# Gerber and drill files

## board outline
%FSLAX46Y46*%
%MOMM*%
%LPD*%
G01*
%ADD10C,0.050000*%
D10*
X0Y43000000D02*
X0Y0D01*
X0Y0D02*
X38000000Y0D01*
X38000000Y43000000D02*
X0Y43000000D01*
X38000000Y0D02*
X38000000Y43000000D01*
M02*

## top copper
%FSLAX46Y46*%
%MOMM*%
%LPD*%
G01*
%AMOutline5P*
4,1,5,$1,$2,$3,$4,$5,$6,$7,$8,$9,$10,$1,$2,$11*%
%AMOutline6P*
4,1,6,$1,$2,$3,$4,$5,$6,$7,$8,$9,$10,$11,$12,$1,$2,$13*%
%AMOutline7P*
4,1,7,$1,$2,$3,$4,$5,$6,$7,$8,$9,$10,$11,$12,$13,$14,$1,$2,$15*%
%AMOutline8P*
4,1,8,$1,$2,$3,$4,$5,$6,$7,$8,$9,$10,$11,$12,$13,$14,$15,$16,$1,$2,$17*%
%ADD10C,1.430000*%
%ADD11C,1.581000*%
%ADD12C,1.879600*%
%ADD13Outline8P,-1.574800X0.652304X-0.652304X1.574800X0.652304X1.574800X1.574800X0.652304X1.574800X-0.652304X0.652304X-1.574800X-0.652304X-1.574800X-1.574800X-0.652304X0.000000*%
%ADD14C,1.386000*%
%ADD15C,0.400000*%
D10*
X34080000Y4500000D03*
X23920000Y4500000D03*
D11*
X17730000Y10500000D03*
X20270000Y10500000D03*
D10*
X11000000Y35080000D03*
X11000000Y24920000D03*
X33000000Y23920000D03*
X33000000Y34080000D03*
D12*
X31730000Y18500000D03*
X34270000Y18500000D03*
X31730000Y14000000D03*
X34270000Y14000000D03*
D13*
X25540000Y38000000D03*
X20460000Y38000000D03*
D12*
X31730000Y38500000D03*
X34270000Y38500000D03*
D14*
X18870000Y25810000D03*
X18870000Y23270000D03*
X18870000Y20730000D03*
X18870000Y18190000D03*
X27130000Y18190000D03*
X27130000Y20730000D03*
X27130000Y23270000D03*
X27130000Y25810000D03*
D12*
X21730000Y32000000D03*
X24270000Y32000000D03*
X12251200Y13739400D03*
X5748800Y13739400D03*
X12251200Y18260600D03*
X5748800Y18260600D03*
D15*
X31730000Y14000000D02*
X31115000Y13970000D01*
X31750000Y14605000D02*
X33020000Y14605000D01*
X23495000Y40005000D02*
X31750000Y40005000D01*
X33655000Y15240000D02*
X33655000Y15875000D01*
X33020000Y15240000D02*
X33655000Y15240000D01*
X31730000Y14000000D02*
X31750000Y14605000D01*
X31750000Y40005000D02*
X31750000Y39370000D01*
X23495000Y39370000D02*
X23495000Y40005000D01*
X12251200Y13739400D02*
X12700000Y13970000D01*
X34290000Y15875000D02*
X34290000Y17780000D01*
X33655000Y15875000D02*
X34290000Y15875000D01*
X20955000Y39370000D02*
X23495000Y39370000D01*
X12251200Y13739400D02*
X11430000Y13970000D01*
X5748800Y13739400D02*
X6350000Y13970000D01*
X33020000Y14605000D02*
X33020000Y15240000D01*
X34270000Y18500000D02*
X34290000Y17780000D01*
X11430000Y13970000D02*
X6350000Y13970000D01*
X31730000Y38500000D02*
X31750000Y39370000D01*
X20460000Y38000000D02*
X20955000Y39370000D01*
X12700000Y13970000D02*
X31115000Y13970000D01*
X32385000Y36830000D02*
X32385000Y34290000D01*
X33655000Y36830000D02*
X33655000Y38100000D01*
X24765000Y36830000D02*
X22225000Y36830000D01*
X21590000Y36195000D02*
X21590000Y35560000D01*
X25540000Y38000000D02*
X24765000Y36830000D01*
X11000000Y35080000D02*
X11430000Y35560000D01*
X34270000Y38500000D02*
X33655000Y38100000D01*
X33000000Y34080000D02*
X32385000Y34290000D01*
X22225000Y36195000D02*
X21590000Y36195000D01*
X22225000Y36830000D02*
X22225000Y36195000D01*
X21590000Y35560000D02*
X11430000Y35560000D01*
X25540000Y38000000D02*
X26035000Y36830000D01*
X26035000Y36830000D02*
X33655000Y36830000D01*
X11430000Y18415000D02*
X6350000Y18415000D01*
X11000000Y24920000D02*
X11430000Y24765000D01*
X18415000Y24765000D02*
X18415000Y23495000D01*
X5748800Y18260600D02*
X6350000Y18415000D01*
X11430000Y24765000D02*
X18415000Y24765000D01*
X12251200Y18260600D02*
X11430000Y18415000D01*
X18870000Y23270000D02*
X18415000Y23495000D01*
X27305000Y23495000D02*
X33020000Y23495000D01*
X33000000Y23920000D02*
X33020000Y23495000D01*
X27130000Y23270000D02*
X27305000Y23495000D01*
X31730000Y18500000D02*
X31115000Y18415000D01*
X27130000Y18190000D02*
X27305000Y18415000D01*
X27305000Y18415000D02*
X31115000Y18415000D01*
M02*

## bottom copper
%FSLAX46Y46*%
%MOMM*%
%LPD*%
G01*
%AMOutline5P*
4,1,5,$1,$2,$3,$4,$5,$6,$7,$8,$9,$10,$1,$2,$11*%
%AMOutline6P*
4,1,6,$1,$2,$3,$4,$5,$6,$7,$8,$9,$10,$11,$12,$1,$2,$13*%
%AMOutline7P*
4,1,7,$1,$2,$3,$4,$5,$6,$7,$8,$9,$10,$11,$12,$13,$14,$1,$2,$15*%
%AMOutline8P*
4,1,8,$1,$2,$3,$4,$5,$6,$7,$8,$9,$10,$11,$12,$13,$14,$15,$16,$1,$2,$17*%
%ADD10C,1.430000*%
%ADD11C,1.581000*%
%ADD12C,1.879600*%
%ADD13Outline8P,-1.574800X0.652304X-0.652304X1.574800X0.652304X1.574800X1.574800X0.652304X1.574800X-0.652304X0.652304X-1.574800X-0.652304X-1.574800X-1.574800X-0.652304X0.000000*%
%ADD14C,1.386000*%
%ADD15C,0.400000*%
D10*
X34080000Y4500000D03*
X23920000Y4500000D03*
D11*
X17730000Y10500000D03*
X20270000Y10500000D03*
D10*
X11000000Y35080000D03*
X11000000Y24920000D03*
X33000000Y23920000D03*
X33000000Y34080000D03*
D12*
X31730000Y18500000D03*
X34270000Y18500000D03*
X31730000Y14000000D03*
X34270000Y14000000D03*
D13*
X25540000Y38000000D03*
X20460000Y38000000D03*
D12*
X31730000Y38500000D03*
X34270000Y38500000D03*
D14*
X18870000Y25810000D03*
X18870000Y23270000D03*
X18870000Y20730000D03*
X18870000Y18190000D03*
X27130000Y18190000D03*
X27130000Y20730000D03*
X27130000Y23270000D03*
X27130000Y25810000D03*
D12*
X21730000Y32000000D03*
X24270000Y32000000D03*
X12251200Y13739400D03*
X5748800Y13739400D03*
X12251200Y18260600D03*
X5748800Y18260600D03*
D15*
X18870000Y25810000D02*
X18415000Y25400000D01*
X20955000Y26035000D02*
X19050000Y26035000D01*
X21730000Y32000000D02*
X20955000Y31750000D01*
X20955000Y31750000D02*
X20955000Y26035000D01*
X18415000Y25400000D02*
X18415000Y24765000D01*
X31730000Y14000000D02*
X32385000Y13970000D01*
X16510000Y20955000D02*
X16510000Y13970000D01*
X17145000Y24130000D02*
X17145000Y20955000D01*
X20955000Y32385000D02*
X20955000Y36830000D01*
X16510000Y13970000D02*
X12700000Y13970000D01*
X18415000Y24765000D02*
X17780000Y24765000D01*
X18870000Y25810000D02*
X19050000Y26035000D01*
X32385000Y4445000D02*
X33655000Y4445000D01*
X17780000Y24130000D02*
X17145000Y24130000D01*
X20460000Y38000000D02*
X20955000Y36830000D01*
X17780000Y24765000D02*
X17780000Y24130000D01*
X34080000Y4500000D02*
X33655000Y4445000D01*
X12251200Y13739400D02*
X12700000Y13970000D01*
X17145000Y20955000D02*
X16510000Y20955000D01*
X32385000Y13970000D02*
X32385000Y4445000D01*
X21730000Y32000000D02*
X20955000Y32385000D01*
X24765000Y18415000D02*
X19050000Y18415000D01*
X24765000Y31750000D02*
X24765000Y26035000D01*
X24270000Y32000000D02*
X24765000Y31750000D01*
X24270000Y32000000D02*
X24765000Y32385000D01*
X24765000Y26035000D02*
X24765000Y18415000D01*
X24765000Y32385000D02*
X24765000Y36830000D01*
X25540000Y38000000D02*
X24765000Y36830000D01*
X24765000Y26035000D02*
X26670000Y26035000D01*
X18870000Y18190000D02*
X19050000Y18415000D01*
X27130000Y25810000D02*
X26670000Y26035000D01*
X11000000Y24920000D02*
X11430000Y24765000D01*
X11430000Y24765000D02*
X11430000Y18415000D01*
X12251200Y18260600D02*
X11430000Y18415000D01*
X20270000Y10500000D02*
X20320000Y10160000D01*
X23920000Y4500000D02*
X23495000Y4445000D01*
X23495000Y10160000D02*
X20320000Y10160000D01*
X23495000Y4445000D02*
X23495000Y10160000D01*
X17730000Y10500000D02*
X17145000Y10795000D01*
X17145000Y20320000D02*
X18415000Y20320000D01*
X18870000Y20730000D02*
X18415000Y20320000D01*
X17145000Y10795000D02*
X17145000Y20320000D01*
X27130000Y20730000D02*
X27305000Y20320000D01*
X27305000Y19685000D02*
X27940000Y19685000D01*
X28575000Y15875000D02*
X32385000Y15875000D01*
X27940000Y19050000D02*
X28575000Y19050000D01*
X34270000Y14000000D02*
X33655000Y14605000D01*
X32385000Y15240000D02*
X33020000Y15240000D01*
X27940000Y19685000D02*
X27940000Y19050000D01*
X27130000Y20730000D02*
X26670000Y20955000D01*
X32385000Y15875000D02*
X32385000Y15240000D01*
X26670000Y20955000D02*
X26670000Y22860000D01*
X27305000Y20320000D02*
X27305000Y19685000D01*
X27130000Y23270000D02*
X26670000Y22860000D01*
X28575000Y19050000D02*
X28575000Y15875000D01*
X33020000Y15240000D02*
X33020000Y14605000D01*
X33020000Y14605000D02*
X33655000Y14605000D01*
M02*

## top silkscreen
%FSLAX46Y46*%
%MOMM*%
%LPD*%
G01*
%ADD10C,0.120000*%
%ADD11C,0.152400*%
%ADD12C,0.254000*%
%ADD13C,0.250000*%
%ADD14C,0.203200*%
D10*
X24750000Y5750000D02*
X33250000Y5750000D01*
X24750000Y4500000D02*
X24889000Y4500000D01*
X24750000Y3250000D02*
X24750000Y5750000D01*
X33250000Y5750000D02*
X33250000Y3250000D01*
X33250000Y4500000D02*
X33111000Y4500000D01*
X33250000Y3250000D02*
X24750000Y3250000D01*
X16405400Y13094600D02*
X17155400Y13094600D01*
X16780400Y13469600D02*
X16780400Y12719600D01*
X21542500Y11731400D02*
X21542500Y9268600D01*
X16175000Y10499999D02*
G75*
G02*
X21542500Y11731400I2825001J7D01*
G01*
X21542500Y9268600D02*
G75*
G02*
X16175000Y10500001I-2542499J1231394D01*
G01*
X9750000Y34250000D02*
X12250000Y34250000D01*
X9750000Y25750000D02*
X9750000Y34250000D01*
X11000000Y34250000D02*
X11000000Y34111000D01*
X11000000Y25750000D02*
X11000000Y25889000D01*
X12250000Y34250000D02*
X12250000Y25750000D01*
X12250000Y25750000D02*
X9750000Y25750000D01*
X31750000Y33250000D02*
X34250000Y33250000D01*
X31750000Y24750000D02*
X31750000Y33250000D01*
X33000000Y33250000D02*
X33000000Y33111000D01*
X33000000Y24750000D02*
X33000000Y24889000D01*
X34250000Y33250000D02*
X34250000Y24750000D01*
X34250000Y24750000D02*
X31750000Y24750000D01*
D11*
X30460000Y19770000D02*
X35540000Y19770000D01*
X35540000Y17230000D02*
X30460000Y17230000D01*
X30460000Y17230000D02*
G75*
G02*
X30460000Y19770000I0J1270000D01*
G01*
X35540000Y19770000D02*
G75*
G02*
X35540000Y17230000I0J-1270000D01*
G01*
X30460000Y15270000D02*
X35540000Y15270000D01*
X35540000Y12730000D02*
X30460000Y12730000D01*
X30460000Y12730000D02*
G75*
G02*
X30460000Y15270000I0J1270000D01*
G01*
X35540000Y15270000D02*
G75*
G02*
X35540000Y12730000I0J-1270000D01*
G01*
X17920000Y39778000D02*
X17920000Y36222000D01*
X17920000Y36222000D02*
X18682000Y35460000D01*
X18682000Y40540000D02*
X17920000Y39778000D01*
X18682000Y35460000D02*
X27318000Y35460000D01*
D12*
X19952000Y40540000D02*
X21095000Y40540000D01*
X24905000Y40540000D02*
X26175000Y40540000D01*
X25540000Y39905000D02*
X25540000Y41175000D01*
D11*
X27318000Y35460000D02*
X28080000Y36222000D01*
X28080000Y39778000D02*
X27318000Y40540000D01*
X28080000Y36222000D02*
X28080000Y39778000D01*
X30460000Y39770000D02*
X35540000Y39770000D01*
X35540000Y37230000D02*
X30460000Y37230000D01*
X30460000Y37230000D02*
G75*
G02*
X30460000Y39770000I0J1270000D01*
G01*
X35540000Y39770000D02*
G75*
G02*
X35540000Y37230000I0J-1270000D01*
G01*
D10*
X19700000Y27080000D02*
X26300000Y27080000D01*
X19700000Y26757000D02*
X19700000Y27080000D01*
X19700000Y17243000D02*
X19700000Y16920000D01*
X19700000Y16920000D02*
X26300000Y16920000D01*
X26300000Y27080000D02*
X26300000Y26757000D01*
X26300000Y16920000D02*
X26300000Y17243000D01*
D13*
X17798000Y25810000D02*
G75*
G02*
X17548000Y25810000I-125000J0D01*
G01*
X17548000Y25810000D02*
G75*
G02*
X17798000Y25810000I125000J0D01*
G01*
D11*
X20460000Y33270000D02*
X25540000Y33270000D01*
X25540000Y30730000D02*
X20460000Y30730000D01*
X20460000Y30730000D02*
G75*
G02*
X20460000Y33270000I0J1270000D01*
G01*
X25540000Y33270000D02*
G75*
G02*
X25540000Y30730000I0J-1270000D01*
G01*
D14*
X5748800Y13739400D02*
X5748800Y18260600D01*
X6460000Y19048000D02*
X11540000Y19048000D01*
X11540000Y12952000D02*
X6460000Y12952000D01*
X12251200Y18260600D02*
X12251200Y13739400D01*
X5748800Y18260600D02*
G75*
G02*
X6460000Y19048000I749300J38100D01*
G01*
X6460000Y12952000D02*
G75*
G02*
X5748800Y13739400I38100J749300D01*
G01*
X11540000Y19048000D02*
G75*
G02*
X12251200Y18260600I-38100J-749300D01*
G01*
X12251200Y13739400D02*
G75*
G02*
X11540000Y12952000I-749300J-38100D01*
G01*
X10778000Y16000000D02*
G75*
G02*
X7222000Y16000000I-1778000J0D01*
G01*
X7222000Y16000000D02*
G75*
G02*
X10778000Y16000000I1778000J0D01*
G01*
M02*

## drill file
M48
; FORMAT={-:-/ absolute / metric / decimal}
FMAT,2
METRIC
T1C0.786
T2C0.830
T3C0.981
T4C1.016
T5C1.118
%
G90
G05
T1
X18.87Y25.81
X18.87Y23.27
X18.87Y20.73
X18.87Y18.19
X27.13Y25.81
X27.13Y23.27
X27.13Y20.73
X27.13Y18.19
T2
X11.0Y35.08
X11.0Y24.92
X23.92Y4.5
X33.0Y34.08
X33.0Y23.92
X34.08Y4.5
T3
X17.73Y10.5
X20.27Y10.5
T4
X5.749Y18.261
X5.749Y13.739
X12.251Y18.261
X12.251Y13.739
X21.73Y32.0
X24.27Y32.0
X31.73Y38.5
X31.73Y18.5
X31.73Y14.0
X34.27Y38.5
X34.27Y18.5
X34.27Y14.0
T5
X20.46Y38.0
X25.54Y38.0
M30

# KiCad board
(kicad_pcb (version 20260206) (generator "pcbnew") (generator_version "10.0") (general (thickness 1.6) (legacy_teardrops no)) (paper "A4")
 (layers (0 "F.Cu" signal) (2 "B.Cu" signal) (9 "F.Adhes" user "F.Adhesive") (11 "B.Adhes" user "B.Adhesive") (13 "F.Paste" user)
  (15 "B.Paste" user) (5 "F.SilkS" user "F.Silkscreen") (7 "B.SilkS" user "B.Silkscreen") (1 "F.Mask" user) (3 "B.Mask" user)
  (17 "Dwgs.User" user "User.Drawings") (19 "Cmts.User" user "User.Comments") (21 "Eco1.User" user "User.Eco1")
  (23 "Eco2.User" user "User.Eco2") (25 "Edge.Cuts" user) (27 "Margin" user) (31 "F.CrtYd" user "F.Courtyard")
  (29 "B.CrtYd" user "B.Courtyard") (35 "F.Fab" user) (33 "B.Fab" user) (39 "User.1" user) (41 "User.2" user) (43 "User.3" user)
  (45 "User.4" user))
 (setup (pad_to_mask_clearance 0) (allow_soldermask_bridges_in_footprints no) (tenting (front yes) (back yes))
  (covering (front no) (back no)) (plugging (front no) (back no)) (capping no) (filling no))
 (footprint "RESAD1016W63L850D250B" (layer "F.Cu") (at 29 -4.5 180)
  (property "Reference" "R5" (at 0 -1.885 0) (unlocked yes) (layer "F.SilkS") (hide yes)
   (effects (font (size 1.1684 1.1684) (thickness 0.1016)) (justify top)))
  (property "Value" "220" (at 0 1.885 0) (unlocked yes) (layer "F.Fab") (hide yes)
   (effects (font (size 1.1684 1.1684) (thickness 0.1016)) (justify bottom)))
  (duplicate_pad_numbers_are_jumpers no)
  (fp_line (start 4.25 1.25) (end -4.25 1.25) (stroke (width 0.12) (type solid)) (layer "F.SilkS"))
  (fp_line (start 4.25 0) (end 4.111 0) (stroke (width 0.12) (type solid)) (layer "F.SilkS"))
  (fp_line (start 4.25 -1.25) (end 4.25 1.25) (stroke (width 0.12) (type solid)) (layer "F.SilkS"))
  (fp_line (start -4.25 1.25) (end -4.25 -1.25) (stroke (width 0.12) (type solid)) (layer "F.SilkS"))
  (fp_line (start -4.25 0) (end -4.111 0) (stroke (width 0.12) (type solid)) (layer "F.SilkS"))
  (fp_line (start -4.25 -1.25) (end 4.25 -1.25) (stroke (width 0.12) (type solid)) (layer "F.SilkS"))
  (pad "1" thru_hole circle (at -5.08 0 180) (size 1.43 1.43) (drill 0.83) (layers "*.Cu" "*.Mask") (remove_unused_layers no) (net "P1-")
   (solder_mask_margin 0.1016) (thermal_bridge_angle 0))
  (pad "2" thru_hole circle (at 5.08 0 180) (size 1.43 1.43) (drill 0.83) (layers "*.Cu" "*.Mask") (remove_unused_layers no) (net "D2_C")
   (solder_mask_margin 0.1016) (thermal_bridge_angle 0)))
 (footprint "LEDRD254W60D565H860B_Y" (layer "F.Cu") (at 19 -10.5)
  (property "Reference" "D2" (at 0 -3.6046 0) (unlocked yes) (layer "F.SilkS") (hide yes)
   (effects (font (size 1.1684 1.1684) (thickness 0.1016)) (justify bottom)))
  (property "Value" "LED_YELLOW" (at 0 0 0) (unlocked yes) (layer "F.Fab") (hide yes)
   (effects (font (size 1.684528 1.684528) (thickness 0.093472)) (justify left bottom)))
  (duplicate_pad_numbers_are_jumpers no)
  (fp_line (start -2.5946 -2.5946) (end -1.8446 -2.5946) (stroke (width 0.12) (type solid)) (layer "F.SilkS"))
  (fp_line (start -2.2196 -2.9696) (end -2.2196 -2.2196) (stroke (width 0.12) (type solid)) (layer "F.SilkS"))
  (fp_line (start 2.5425 -1.2314) (end 2.5425 1.2314) (stroke (width 0.12) (type solid)) (layer "F.SilkS"))
  (fp_arc (start -2.825 0.000001) (mid -0.631694 -2.753475) (end 2.5425 -1.2314) (stroke (width 0.12) (type solid)) (layer "F.SilkS"))
  (fp_arc (start 2.5425 1.2314) (mid -0.631694 2.753475) (end -2.825 -0.000001) (stroke (width 0.12) (type solid)) (layer "F.SilkS"))
  (pad "1" thru_hole circle (at -1.27 0) (size 1.581 1.581) (drill 0.981) (layers "*.Cu" "*.Mask") (remove_unused_layers no) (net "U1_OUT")
   (solder_mask_margin 0.1016) (thermal_bridge_angle 0))
  (pad "2" thru_hole circle (at 1.27 0) (size 1.581 1.581) (drill 0.981) (layers "*.Cu" "*.Mask") (remove_unused_layers no) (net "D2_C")
   (solder_mask_margin 0.1016) (thermal_bridge_angle 0)))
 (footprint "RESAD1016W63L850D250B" (layer "F.Cu") (at 11 -30 -90)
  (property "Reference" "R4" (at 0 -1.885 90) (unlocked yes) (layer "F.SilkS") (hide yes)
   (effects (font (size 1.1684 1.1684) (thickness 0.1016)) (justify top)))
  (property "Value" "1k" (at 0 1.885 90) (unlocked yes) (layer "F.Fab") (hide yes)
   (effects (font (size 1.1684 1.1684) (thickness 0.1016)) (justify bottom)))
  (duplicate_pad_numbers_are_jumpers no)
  (fp_line (start -4.25 1.25) (end -4.25 -1.25) (stroke (width 0.12) (type solid)) (layer "F.SilkS"))
  (fp_line (start 4.25 1.25) (end -4.25 1.25) (stroke (width 0.12) (type solid)) (layer "F.SilkS"))
  (fp_line (start -4.25 0) (end -4.111 0) (stroke (width 0.12) (type solid)) (layer "F.SilkS"))
  (fp_line (start 4.25 0) (end 4.111 0) (stroke (width 0.12) (type solid)) (layer "F.SilkS"))
  (fp_line (start -4.25 -1.25) (end 4.25 -1.25) (stroke (width 0.12) (type solid)) (layer "F.SilkS"))
  (fp_line (start 4.25 -1.25) (end 4.25 1.25) (stroke (width 0.12) (type solid)) (layer "F.SilkS"))
  (pad "1" thru_hole circle (at -5.08 0 270) (size 1.43 1.43) (drill 0.83) (layers "*.Cu" "*.Mask") (remove_unused_layers no) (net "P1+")
   (solder_mask_margin 0.1016) (thermal_bridge_angle 0))
  (pad "2" thru_hole circle (at 5.08 0 270) (size 1.43 1.43) (drill 0.83) (layers "*.Cu" "*.Mask") (remove_unused_layers no) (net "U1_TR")
   (solder_mask_margin 0.1016) (thermal_bridge_angle 0)))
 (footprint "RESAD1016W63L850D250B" (layer "F.Cu") (at 33 -29 90)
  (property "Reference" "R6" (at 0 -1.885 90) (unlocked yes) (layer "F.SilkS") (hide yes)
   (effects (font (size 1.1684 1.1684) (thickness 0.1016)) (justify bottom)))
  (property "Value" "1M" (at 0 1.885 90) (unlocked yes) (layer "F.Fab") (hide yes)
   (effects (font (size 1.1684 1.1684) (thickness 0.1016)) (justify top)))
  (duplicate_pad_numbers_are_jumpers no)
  (fp_line (start 4.25 -1.25) (end 4.25 1.25) (stroke (width 0.12) (type solid)) (layer "F.SilkS"))
  (fp_line (start -4.25 -1.25) (end 4.25 -1.25) (stroke (width 0.12) (type solid)) (layer "F.SilkS"))
  (fp_line (start 4.25 0) (end 4.111 0) (stroke (width 0.12) (type solid)) (layer "F.SilkS"))
  (fp_line (start -4.25 0) (end -4.111 0) (stroke (width 0.12) (type solid)) (layer "F.SilkS"))
  (fp_line (start 4.25 1.25) (end -4.25 1.25) (stroke (width 0.12) (type solid)) (layer "F.SilkS"))
  (fp_line (start -4.25 1.25) (end -4.25 -1.25) (stroke (width 0.12) (type solid)) (layer "F.SilkS"))
  (pad "1" thru_hole circle (at -5.08 0 90) (size 1.43 1.43) (drill 0.83) (layers "*.Cu" "*.Mask") (remove_unused_layers no) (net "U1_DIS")
   (solder_mask_margin 0.1016) (thermal_bridge_angle 0))
  (pad "2" thru_hole circle (at 5.08 0 90) (size 1.43 1.43) (drill 0.83) (layers "*.Cu" "*.Mask") (remove_unused_layers no) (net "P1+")
   (solder_mask_margin 0.1016) (thermal_bridge_angle 0)))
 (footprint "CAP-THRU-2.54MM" (layer "F.Cu") (at 33 -18.5)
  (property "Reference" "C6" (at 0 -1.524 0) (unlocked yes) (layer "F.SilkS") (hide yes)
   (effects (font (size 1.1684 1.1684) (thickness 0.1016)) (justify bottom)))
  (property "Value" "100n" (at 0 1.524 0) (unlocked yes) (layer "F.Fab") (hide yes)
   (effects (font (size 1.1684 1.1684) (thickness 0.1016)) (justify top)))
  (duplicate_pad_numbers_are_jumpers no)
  (fp_line (start -2.54 -1.27) (end 2.54 -1.27) (stroke (width 0.1524) (type solid)) (layer "F.SilkS"))
  (fp_line (start 2.54 1.27) (end -2.54 1.27) (stroke (width 0.1524) (type solid)) (layer "F.SilkS"))
  (fp_arc (start -2.54 1.27) (mid -3.81 0) (end -2.54 -1.27) (stroke (width 0.1524) (type solid)) (layer "F.SilkS"))
  (fp_arc (start 2.54 -1.27) (mid 3.81 0) (end 2.54 1.27) (stroke (width 0.1524) (type solid)) (layer "F.SilkS"))
  (pad "1" thru_hole circle (at -1.27 0) (size 1.8796 1.8796) (drill 1.016) (layers "*.Cu" "*.Mask") (remove_unused_layers no) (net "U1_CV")
   (solder_mask_margin 0.1016) (thermal_bridge_angle 0))
  (pad "2" thru_hole circle (at 1.27 0) (size 1.8796 1.8796) (drill 1.016) (layers "*.Cu" "*.Mask") (remove_unused_layers no) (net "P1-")
   (solder_mask_margin 0.1016) (thermal_bridge_angle 0)))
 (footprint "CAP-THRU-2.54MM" (layer "F.Cu") (at 33 -14)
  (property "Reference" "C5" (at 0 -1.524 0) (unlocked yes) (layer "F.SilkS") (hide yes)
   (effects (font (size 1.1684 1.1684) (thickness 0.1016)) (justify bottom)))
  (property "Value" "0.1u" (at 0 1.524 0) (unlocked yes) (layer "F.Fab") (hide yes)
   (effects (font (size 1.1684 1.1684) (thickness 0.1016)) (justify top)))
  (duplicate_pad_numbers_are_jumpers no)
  (fp_line (start -2.54 -1.27) (end 2.54 -1.27) (stroke (width 0.1524) (type solid)) (layer "F.SilkS"))
  (fp_line (start 2.54 1.27) (end -2.54 1.27) (stroke (width 0.1524) (type solid)) (layer "F.SilkS"))
  (fp_arc (start -2.54 1.27) (mid -3.81 0) (end -2.54 -1.27) (stroke (width 0.1524) (type solid)) (layer "F.SilkS"))
  (fp_arc (start 2.54 -1.27) (mid 3.81 0) (end 2.54 1.27) (stroke (width 0.1524) (type solid)) (layer "F.SilkS"))
  (pad "1" thru_hole circle (at -1.27 0) (size 1.8796 1.8796) (drill 1.016) (layers "*.Cu" "*.Mask") (remove_unused_layers no) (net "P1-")
   (solder_mask_margin 0.1016) (thermal_bridge_angle 0))
  (pad "2" thru_hole circle (at 1.27 0) (size 1.8796 1.8796) (drill 1.016) (layers "*.Cu" "*.Mask") (remove_unused_layers no) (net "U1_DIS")
   (solder_mask_margin 0.1016) (thermal_bridge_angle 0)))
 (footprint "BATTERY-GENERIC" (layer "F.Cu") (at 23 -38)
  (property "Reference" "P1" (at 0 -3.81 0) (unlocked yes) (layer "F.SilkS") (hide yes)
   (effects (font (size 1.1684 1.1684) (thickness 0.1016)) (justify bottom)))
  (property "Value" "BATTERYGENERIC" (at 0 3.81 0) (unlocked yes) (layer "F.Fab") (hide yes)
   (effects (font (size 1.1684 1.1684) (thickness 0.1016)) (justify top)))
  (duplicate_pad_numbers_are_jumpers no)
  (fp_line (start -5.08 -1.778) (end -5.08 1.778) (stroke (width 0.1524) (type solid)) (layer "F.SilkS"))
  (fp_line (start -5.08 1.778) (end -4.318 2.54) (stroke (width 0.1524) (type solid)) (layer "F.SilkS"))
  (fp_line (start -4.318 -2.54) (end -5.08 -1.778) (stroke (width 0.1524) (type solid)) (layer "F.SilkS"))
  (fp_line (start -4.318 2.54) (end 4.318 2.54) (stroke (width 0.1524) (type solid)) (layer "F.SilkS"))
  (fp_line (start -3.048 -2.54) (end -1.905 -2.54) (stroke (width 0.254) (type solid)) (layer "F.SilkS"))
  (fp_line (start 1.905 -2.54) (end 3.175 -2.54) (stroke (width 0.254) (type solid)) (layer "F.SilkS"))
  (fp_line (start 2.54 -1.905) (end 2.54 -3.175) (stroke (width 0.254) (type solid)) (layer "F.SilkS"))
  (fp_line (start 4.318 2.54) (end 5.08 1.778) (stroke (width 0.1524) (type solid)) (layer "F.SilkS"))
  (fp_line (start 5.08 -1.778) (end 4.318 -2.54) (stroke (width 0.1524) (type solid)) (layer "F.SilkS"))
  (fp_line (start 5.08 1.778) (end 5.08 -1.778) (stroke (width 0.1524) (type solid)) (layer "F.SilkS"))
  (pad "+" thru_hole roundrect (at 2.54 0) (size 3.1496 3.1496) (drill 1.1176) (layers "*.Cu" "*.Mask") (remove_unused_layers no)
   (roundrect_rratio 0.25) (chamfer_ratio 0.2928932188) (chamfer top_left top_right bottom_left bottom_right) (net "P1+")
   (solder_mask_margin 0.1016) (thermal_bridge_angle 0))
  (pad "-" thru_hole roundrect (at -2.54 0) (size 3.1496 3.1496) (drill 1.1176) (layers "*.Cu" "*.Mask") (remove_unused_layers no)
   (roundrect_rratio 0.25) (chamfer_ratio 0.2928932188) (chamfer top_left top_right bottom_left bottom_right) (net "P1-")
   (solder_mask_margin 0.1016) (thermal_bridge_angle 0)))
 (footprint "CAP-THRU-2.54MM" (layer "F.Cu") (at 33 -38.5)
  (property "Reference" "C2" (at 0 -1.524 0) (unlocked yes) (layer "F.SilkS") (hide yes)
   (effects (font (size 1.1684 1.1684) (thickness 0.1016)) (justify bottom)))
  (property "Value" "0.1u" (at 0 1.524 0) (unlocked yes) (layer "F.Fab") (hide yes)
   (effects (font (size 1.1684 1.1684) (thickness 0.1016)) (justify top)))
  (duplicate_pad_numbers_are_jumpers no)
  (fp_line (start -2.54 -1.27) (end 2.54 -1.27) (stroke (width 0.1524) (type solid)) (layer "F.SilkS"))
  (fp_line (start 2.54 1.27) (end -2.54 1.27) (stroke (width 0.1524) (type solid)) (layer "F.SilkS"))
  (fp_arc (start -2.54 1.27) (mid -3.81 0) (end -2.54 -1.27) (stroke (width 0.1524) (type solid)) (layer "F.SilkS"))
  (fp_arc (start 2.54 -1.27) (mid 3.81 0) (end 2.54 1.27) (stroke (width 0.1524) (type solid)) (layer "F.SilkS"))
  (pad "1" thru_hole circle (at -1.27 0) (size 1.8796 1.8796) (drill 1.016) (layers "*.Cu" "*.Mask") (remove_unused_layers no) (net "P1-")
   (solder_mask_margin 0.1016) (thermal_bridge_angle 0))
  (pad "2" thru_hole circle (at 1.27 0) (size 1.8796 1.8796) (drill 1.016) (layers "*.Cu" "*.Mask") (remove_unused_layers no) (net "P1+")
   (solder_mask_margin 0.1016) (thermal_bridge_angle 0)))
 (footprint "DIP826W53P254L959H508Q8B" (layer "F.Cu") (at 23 -22)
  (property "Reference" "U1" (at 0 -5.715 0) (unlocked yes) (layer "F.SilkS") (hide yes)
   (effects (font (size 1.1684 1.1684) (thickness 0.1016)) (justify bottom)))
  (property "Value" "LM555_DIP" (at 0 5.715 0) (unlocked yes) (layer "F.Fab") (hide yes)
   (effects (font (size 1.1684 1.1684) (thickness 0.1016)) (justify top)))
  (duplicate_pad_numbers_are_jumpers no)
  (fp_line (start -3.3 -5.08) (end 3.3 -5.08) (stroke (width 0.12) (type solid)) (layer "F.SilkS"))
  (fp_line (start -3.3 -4.757) (end -3.3 -5.08) (stroke (width 0.12) (type solid)) (layer "F.SilkS"))
  (fp_line (start -3.3 4.757) (end -3.3 5.08) (stroke (width 0.12) (type solid)) (layer "F.SilkS"))
  (fp_line (start -3.3 5.08) (end 3.3 5.08) (stroke (width 0.12) (type solid)) (layer "F.SilkS"))
  (fp_line (start 3.3 -5.08) (end 3.3 -4.757) (stroke (width 0.12) (type solid)) (layer "F.SilkS"))
  (fp_line (start 3.3 5.08) (end 3.3 4.757) (stroke (width 0.12) (type solid)) (layer "F.SilkS"))
  (fp_circle (center -5.327 -3.81) (end -5.202 -3.81) (stroke (width 0.25) (type solid)) (fill yes) (layer "F.SilkS"))
  (pad "1" thru_hole circle (at -4.13 -3.81) (size 1.386 1.386) (drill 0.786) (layers "*.Cu" "*.Mask") (remove_unused_layers no) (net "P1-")
   (solder_mask_margin 0.1016) (thermal_bridge_angle 0))
  (pad "2" thru_hole circle (at -4.13 -1.27) (size 1.386 1.386) (drill 0.786) (layers "*.Cu" "*.Mask") (remove_unused_layers no)
   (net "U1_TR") (solder_mask_margin 0.1016) (thermal_bridge_angle 0))
  (pad "3" thru_hole circle (at -4.13 1.27) (size 1.386 1.386) (drill 0.786) (layers "*.Cu" "*.Mask") (remove_unused_layers no)
   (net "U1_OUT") (solder_mask_margin 0.1016) (thermal_bridge_angle 0))
  (pad "4" thru_hole circle (at -4.13 3.81) (size 1.386 1.386) (drill 0.786) (layers "*.Cu" "*.Mask") (remove_unused_layers no) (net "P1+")
   (solder_mask_margin 0.1016) (thermal_bridge_angle 0))
  (pad "5" thru_hole circle (at 4.13 3.81) (size 1.386 1.386) (drill 0.786) (layers "*.Cu" "*.Mask") (remove_unused_layers no) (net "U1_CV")
   (solder_mask_margin 0.1016) (thermal_bridge_angle 0))
  (pad "6" thru_hole circle (at 4.13 1.27) (size 1.386 1.386) (drill 0.786) (layers "*.Cu" "*.Mask") (remove_unused_layers no)
   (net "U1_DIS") (solder_mask_margin 0.1016) (thermal_bridge_angle 0))
  (pad "7" thru_hole circle (at 4.13 -1.27) (size 1.386 1.386) (drill 0.786) (layers "*.Cu" "*.Mask") (remove_unused_layers no)
   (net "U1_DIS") (solder_mask_margin 0.1016) (thermal_bridge_angle 0))
  (pad "8" thru_hole circle (at 4.13 -3.81) (size 1.386 1.386) (drill 0.786) (layers "*.Cu" "*.Mask") (remove_unused_layers no) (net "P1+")
   (solder_mask_margin 0.1016) (thermal_bridge_angle 0)))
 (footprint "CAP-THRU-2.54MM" (layer "F.Cu") (at 23 -32)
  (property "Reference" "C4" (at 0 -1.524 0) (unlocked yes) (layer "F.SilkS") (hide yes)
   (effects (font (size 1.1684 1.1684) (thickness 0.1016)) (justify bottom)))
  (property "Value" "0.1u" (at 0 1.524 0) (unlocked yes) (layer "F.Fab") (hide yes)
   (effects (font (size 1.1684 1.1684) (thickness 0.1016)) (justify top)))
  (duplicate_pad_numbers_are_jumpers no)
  (fp_line (start -2.54 -1.27) (end 2.54 -1.27) (stroke (width 0.1524) (type solid)) (layer "F.SilkS"))
  (fp_line (start 2.54 1.27) (end -2.54 1.27) (stroke (width 0.1524) (type solid)) (layer "F.SilkS"))
  (fp_arc (start -2.54 1.27) (mid -3.81 0) (end -2.54 -1.27) (stroke (width 0.1524) (type solid)) (layer "F.SilkS"))
  (fp_arc (start 2.54 -1.27) (mid 3.81 0) (end 2.54 1.27) (stroke (width 0.1524) (type solid)) (layer "F.SilkS"))
  (pad "1" thru_hole circle (at -1.27 0) (size 1.8796 1.8796) (drill 1.016) (layers "*.Cu" "*.Mask") (remove_unused_layers no) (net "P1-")
   (solder_mask_margin 0.1016) (thermal_bridge_angle 0))
  (pad "2" thru_hole circle (at 1.27 0) (size 1.8796 1.8796) (drill 1.016) (layers "*.Cu" "*.Mask") (remove_unused_layers no) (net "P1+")
   (solder_mask_margin 0.1016) (thermal_bridge_angle 0)))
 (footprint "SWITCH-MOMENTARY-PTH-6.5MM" (layer "F.Cu") (at 9 -16 180)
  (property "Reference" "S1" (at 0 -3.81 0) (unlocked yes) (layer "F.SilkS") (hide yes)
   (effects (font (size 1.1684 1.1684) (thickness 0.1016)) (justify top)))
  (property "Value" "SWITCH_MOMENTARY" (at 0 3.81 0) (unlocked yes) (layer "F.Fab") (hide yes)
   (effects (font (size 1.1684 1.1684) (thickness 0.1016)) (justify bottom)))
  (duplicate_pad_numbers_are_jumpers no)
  (fp_line (start 3.2512 -2.2606) (end 3.2512 2.2606) (stroke (width 0.2032) (type solid)) (layer "F.SilkS"))
  (fp_line (start 2.54 3.048) (end -2.54 3.048) (stroke (width 0.2032) (type solid)) (layer "F.SilkS"))
  (fp_line (start -2.54 -3.048) (end 2.54 -3.048) (stroke (width 0.2032) (type solid)) (layer "F.SilkS"))
  (fp_line (start -3.2512 2.2606) (end -3.2512 -2.2606) (stroke (width 0.2032) (type solid)) (layer "F.SilkS"))
  (fp_arc (start 3.2512 2.2606) (mid 3.058676 2.801594) (end 2.54 3.048) (stroke (width 0.2032) (type solid)) (layer "F.SilkS"))
  (fp_arc (start 2.54 -3.048) (mid 3.058676 -2.801594) (end 3.2512 -2.2606) (stroke (width 0.2032) (type solid)) (layer "F.SilkS"))
  (fp_arc (start -2.54 3.048) (mid -3.058676 2.801594) (end -3.2512 2.2606) (stroke (width 0.2032) (type solid)) (layer "F.SilkS"))
  (fp_arc (start -3.2512 -2.2606) (mid -3.058676 -2.801594) (end -2.54 -3.048) (stroke (width 0.2032) (type solid)) (layer "F.SilkS"))
  (fp_circle (center 0 0) (end 1.778 0) (stroke (width 0.2032) (type solid)) (fill no) (layer "F.SilkS"))
  (pad "1" thru_hole circle (at -3.2512 -2.2606 180) (size 1.8796 1.8796) (drill 1.016) (layers "*.Cu" "*.Mask") (remove_unused_layers no)
   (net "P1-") (solder_mask_margin 0.1016) (thermal_bridge_angle 0))
  (pad "2" thru_hole circle (at 3.2512 -2.2606 180) (size 1.8796 1.8796) (drill 1.016) (layers "*.Cu" "*.Mask") (remove_unused_layers no)
   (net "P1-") (solder_mask_margin 0.1016) (thermal_bridge_angle 0))
  (pad "3" thru_hole circle (at -3.2512 2.2606 180) (size 1.8796 1.8796) (drill 1.016) (layers "*.Cu" "*.Mask") (remove_unused_layers no)
   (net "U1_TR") (solder_mask_margin 0.1016) (thermal_bridge_angle 0))
  (pad "4" thru_hole circle (at 3.2512 2.2606 180) (size 1.8796 1.8796) (drill 1.016) (layers "*.Cu" "*.Mask") (remove_unused_layers no)
   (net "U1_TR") (solder_mask_margin 0.1016) (thermal_bridge_angle 0)))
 (gr_line (start 0 -43) (end 0 0) (stroke (width 0.05) (type solid)) (layer "Edge.Cuts"))
 (gr_line (start 0 0) (end 38 0) (stroke (width 0.05) (type solid)) (layer "Edge.Cuts"))
 (gr_line (start 38 -43) (end 0 -43) (stroke (width 0.05) (type solid)) (layer "Edge.Cuts"))
 (gr_line (start 38 0) (end 38 -43) (stroke (width 0.05) (type solid)) (layer "Edge.Cuts"))
 (segment (start 31.73 -14) (end 31.115 -13.97) (width 0.4) (layer "F.Cu") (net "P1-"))
 (segment (start 31.75 -14.605) (end 33.02 -14.605) (width 0.4) (layer "F.Cu") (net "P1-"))
 (segment (start 23.495 -40.005) (end 31.75 -40.005) (width 0.4) (layer "F.Cu") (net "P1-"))
 (segment (start 33.655 -15.24) (end 33.655 -15.875) (width 0.4) (layer "F.Cu") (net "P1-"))
 (segment (start 33.02 -15.24) (end 33.655 -15.24) (width 0.4) (layer "F.Cu") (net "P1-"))
 (segment (start 31.73 -14) (end 31.75 -14.605) (width 0.4) (layer "F.Cu") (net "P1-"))
 (segment (start 31.75 -40.005) (end 31.75 -39.37) (width 0.4) (layer "F.Cu") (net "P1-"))
 (segment (start 23.495 -39.37) (end 23.495 -40.005) (width 0.4) (layer "F.Cu") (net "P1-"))
 (segment (start 12.2512 -13.7394) (end 12.7 -13.97) (width 0.4) (layer "F.Cu") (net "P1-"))
 (segment (start 34.29 -15.875) (end 34.29 -17.78) (width 0.4) (layer "F.Cu") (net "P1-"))
 (segment (start 33.655 -15.875) (end 34.29 -15.875) (width 0.4) (layer "F.Cu") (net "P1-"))
 (segment (start 20.955 -39.37) (end 23.495 -39.37) (width 0.4) (layer "F.Cu") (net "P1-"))
 (segment (start 12.2512 -13.7394) (end 11.43 -13.97) (width 0.4) (layer "F.Cu") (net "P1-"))
 (segment (start 5.7488 -13.7394) (end 6.35 -13.97) (width 0.4) (layer "F.Cu") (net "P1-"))
 (segment (start 33.02 -14.605) (end 33.02 -15.24) (width 0.4) (layer "F.Cu") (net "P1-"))
 (segment (start 34.27 -18.5) (end 34.29 -17.78) (width 0.4) (layer "F.Cu") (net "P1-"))
 (segment (start 11.43 -13.97) (end 6.35 -13.97) (width 0.4) (layer "F.Cu") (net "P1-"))
 (segment (start 31.73 -38.5) (end 31.75 -39.37) (width 0.4) (layer "F.Cu") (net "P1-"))
 (segment (start 20.46 -38) (end 20.955 -39.37) (width 0.4) (layer "F.Cu") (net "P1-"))
 (segment (start 12.7 -13.97) (end 31.115 -13.97) (width 0.4) (layer "F.Cu") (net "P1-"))
 (segment (start 18.87 -25.81) (end 18.415 -25.4) (width 0.4) (layer "B.Cu") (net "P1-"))
 (segment (start 20.955 -26.035) (end 19.05 -26.035) (width 0.4) (layer "B.Cu") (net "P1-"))
 (segment (start 21.73 -32) (end 20.955 -31.75) (width 0.4) (layer "B.Cu") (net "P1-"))
 (segment (start 20.955 -31.75) (end 20.955 -26.035) (width 0.4) (layer "B.Cu") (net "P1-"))
 (segment (start 18.415 -25.4) (end 18.415 -24.765) (width 0.4) (layer "B.Cu") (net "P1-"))
 (segment (start 31.73 -14) (end 32.385 -13.97) (width 0.4) (layer "B.Cu") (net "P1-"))
 (segment (start 16.51 -20.955) (end 16.51 -13.97) (width 0.4) (layer "B.Cu") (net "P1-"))
 (segment (start 17.145 -24.13) (end 17.145 -20.955) (width 0.4) (layer "B.Cu") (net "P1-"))
 (segment (start 20.955 -32.385) (end 20.955 -36.83) (width 0.4) (layer "B.Cu") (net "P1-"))
 (segment (start 16.51 -13.97) (end 12.7 -13.97) (width 0.4) (layer "B.Cu") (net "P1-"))
 (segment (start 18.415 -24.765) (end 17.78 -24.765) (width 0.4) (layer "B.Cu") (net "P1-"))
 (segment (start 18.87 -25.81) (end 19.05 -26.035) (width 0.4) (layer "B.Cu") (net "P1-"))
 (segment (start 32.385 -4.445) (end 33.655 -4.445) (width 0.4) (layer "B.Cu") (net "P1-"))
 (segment (start 17.78 -24.13) (end 17.145 -24.13) (width 0.4) (layer "B.Cu") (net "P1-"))
 (segment (start 20.46 -38) (end 20.955 -36.83) (width 0.4) (layer "B.Cu") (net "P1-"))
 (segment (start 17.78 -24.765) (end 17.78 -24.13) (width 0.4) (layer "B.Cu") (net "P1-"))
 (segment (start 34.08 -4.5) (end 33.655 -4.445) (width 0.4) (layer "B.Cu") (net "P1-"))
 (segment (start 12.2512 -13.7394) (end 12.7 -13.97) (width 0.4) (layer "B.Cu") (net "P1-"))
 (segment (start 17.145 -20.955) (end 16.51 -20.955) (width 0.4) (layer "B.Cu") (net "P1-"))
 (segment (start 32.385 -13.97) (end 32.385 -4.445) (width 0.4) (layer "B.Cu") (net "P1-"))
 (segment (start 21.73 -32) (end 20.955 -32.385) (width 0.4) (layer "B.Cu") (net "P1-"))
 (segment (start 32.385 -36.83) (end 32.385 -34.29) (width 0.4) (layer "F.Cu") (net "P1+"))
 (segment (start 33.655 -36.83) (end 33.655 -38.1) (width 0.4) (layer "F.Cu") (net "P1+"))
 (segment (start 24.765 -36.83) (end 22.225 -36.83) (width 0.4) (layer "F.Cu") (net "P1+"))
 (segment (start 21.59 -36.195) (end 21.59 -35.56) (width 0.4) (layer "F.Cu") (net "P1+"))
 (segment (start 25.54 -38) (end 24.765 -36.83) (width 0.4) (layer "F.Cu") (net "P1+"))
 (segment (start 11 -35.08) (end 11.43 -35.56) (width 0.4) (layer "F.Cu") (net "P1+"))
 (segment (start 34.27 -38.5) (end 33.655 -38.1) (width 0.4) (layer "F.Cu") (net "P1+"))
 (segment (start 33 -34.08) (end 32.385 -34.29) (width 0.4) (layer "F.Cu") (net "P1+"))
 (segment (start 22.225 -36.195) (end 21.59 -36.195) (width 0.4) (layer "F.Cu") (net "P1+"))
 (segment (start 22.225 -36.83) (end 22.225 -36.195) (width 0.4) (layer "F.Cu") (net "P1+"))
 (segment (start 21.59 -35.56) (end 11.43 -35.56) (width 0.4) (layer "F.Cu") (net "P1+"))
 (segment (start 25.54 -38) (end 26.035 -36.83) (width 0.4) (layer "F.Cu") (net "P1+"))
 (segment (start 26.035 -36.83) (end 33.655 -36.83) (width 0.4) (layer "F.Cu") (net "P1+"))
 (segment (start 24.765 -18.415) (end 19.05 -18.415) (width 0.4) (layer "B.Cu") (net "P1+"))
 (segment (start 24.765 -31.75) (end 24.765 -26.035) (width 0.4) (layer "B.Cu") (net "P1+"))
 (segment (start 24.27 -32) (end 24.765 -31.75) (width 0.4) (layer "B.Cu") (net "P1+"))
 (segment (start 24.27 -32) (end 24.765 -32.385) (width 0.4) (layer "B.Cu") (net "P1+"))
 (segment (start 24.765 -26.035) (end 24.765 -18.415) (width 0.4) (layer "B.Cu") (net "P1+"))
 (segment (start 24.765 -32.385) (end 24.765 -36.83) (width 0.4) (layer "B.Cu") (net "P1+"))
 (segment (start 25.54 -38) (end 24.765 -36.83) (width 0.4) (layer "B.Cu") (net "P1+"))
 (segment (start 24.765 -26.035) (end 26.67 -26.035) (width 0.4) (layer "B.Cu") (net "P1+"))
 (segment (start 18.87 -18.19) (end 19.05 -18.415) (width 0.4) (layer "B.Cu") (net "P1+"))
 (segment (start 27.13 -25.81) (end 26.67 -26.035) (width 0.4) (layer "B.Cu") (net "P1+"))
 (segment (start 11.43 -18.415) (end 6.35 -18.415) (width 0.4) (layer "F.Cu") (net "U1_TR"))
 (segment (start 11 -24.92) (end 11.43 -24.765) (width 0.4) (layer "F.Cu") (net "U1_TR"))
 (segment (start 18.415 -24.765) (end 18.415 -23.495) (width 0.4) (layer "F.Cu") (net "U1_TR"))
 (segment (start 5.7488 -18.2606) (end 6.35 -18.415) (width 0.4) (layer "F.Cu") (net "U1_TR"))
 (segment (start 11.43 -24.765) (end 18.415 -24.765) (width 0.4) (layer "F.Cu") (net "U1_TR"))
 (segment (start 12.2512 -18.2606) (end 11.43 -18.415) (width 0.4) (layer "F.Cu") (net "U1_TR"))
 (segment (start 18.87 -23.27) (end 18.415 -23.495) (width 0.4) (layer "F.Cu") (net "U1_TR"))
 (segment (start 11 -24.92) (end 11.43 -24.765) (width 0.4) (layer "B.Cu") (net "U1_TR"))
 (segment (start 11.43 -24.765) (end 11.43 -18.415) (width 0.4) (layer "B.Cu") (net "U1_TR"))
 (segment (start 12.2512 -18.2606) (end 11.43 -18.415) (width 0.4) (layer "B.Cu") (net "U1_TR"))
 (segment (start 20.27 -10.5) (end 20.32 -10.16) (width 0.4) (layer "B.Cu") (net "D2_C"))
 (segment (start 23.92 -4.5) (end 23.495 -4.445) (width 0.4) (layer "B.Cu") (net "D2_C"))
 (segment (start 23.495 -10.16) (end 20.32 -10.16) (width 0.4) (layer "B.Cu") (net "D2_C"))
 (segment (start 23.495 -4.445) (end 23.495 -10.16) (width 0.4) (layer "B.Cu") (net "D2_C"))
 (segment (start 17.73 -10.5) (end 17.145 -10.795) (width 0.4) (layer "B.Cu") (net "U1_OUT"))
 (segment (start 17.145 -20.32) (end 18.415 -20.32) (width 0.4) (layer "B.Cu") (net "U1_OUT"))
 (segment (start 18.87 -20.73) (end 18.415 -20.32) (width 0.4) (layer "B.Cu") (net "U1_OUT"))
 (segment (start 17.145 -10.795) (end 17.145 -20.32) (width 0.4) (layer "B.Cu") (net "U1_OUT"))
 (segment (start 27.305 -23.495) (end 33.02 -23.495) (width 0.4) (layer "F.Cu") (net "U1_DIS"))
 (segment (start 33 -23.92) (end 33.02 -23.495) (width 0.4) (layer "F.Cu") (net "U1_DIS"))
 (segment (start 27.13 -23.27) (end 27.305 -23.495) (width 0.4) (layer "F.Cu") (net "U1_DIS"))
 (segment (start 27.13 -20.73) (end 27.305 -20.32) (width 0.4) (layer "B.Cu") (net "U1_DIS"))
 (segment (start 27.305 -19.685) (end 27.94 -19.685) (width 0.4) (layer "B.Cu") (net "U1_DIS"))
 (segment (start 28.575 -15.875) (end 32.385 -15.875) (width 0.4) (layer "B.Cu") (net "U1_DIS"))
 (segment (start 27.94 -19.05) (end 28.575 -19.05) (width 0.4) (layer "B.Cu") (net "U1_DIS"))
 (segment (start 34.27 -14) (end 33.655 -14.605) (width 0.4) (layer "B.Cu") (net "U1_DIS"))
 (segment (start 32.385 -15.24) (end 33.02 -15.24) (width 0.4) (layer "B.Cu") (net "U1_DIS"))
 (segment (start 27.94 -19.685) (end 27.94 -19.05) (width 0.4) (layer "B.Cu") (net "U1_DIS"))
 (segment (start 27.13 -20.73) (end 26.67 -20.955) (width 0.4) (layer "B.Cu") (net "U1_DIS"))
 (segment (start 32.385 -15.875) (end 32.385 -15.24) (width 0.4) (layer "B.Cu") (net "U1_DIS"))
 (segment (start 26.67 -20.955) (end 26.67 -22.86) (width 0.4) (layer "B.Cu") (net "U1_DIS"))
 (segment (start 27.305 -20.32) (end 27.305 -19.685) (width 0.4) (layer "B.Cu") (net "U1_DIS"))
 (segment (start 27.13 -23.27) (end 26.67 -22.86) (width 0.4) (layer "B.Cu") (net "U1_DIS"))
 (segment (start 28.575 -19.05) (end 28.575 -15.875) (width 0.4) (layer "B.Cu") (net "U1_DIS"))
 (segment (start 33.02 -15.24) (end 33.02 -14.605) (width 0.4) (layer "B.Cu") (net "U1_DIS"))
 (segment (start 33.02 -14.605) (end 33.655 -14.605) (width 0.4) (layer "B.Cu") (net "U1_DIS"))
 (segment (start 31.73 -18.5) (end 31.115 -18.415) (width 0.4) (layer "F.Cu") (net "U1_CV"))
 (segment (start 27.13 -18.19) (end 27.305 -18.415) (width 0.4) (layer "F.Cu") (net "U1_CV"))
 (segment (start 27.305 -18.415) (end 31.115 -18.415) (width 0.4) (layer "F.Cu") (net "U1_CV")))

